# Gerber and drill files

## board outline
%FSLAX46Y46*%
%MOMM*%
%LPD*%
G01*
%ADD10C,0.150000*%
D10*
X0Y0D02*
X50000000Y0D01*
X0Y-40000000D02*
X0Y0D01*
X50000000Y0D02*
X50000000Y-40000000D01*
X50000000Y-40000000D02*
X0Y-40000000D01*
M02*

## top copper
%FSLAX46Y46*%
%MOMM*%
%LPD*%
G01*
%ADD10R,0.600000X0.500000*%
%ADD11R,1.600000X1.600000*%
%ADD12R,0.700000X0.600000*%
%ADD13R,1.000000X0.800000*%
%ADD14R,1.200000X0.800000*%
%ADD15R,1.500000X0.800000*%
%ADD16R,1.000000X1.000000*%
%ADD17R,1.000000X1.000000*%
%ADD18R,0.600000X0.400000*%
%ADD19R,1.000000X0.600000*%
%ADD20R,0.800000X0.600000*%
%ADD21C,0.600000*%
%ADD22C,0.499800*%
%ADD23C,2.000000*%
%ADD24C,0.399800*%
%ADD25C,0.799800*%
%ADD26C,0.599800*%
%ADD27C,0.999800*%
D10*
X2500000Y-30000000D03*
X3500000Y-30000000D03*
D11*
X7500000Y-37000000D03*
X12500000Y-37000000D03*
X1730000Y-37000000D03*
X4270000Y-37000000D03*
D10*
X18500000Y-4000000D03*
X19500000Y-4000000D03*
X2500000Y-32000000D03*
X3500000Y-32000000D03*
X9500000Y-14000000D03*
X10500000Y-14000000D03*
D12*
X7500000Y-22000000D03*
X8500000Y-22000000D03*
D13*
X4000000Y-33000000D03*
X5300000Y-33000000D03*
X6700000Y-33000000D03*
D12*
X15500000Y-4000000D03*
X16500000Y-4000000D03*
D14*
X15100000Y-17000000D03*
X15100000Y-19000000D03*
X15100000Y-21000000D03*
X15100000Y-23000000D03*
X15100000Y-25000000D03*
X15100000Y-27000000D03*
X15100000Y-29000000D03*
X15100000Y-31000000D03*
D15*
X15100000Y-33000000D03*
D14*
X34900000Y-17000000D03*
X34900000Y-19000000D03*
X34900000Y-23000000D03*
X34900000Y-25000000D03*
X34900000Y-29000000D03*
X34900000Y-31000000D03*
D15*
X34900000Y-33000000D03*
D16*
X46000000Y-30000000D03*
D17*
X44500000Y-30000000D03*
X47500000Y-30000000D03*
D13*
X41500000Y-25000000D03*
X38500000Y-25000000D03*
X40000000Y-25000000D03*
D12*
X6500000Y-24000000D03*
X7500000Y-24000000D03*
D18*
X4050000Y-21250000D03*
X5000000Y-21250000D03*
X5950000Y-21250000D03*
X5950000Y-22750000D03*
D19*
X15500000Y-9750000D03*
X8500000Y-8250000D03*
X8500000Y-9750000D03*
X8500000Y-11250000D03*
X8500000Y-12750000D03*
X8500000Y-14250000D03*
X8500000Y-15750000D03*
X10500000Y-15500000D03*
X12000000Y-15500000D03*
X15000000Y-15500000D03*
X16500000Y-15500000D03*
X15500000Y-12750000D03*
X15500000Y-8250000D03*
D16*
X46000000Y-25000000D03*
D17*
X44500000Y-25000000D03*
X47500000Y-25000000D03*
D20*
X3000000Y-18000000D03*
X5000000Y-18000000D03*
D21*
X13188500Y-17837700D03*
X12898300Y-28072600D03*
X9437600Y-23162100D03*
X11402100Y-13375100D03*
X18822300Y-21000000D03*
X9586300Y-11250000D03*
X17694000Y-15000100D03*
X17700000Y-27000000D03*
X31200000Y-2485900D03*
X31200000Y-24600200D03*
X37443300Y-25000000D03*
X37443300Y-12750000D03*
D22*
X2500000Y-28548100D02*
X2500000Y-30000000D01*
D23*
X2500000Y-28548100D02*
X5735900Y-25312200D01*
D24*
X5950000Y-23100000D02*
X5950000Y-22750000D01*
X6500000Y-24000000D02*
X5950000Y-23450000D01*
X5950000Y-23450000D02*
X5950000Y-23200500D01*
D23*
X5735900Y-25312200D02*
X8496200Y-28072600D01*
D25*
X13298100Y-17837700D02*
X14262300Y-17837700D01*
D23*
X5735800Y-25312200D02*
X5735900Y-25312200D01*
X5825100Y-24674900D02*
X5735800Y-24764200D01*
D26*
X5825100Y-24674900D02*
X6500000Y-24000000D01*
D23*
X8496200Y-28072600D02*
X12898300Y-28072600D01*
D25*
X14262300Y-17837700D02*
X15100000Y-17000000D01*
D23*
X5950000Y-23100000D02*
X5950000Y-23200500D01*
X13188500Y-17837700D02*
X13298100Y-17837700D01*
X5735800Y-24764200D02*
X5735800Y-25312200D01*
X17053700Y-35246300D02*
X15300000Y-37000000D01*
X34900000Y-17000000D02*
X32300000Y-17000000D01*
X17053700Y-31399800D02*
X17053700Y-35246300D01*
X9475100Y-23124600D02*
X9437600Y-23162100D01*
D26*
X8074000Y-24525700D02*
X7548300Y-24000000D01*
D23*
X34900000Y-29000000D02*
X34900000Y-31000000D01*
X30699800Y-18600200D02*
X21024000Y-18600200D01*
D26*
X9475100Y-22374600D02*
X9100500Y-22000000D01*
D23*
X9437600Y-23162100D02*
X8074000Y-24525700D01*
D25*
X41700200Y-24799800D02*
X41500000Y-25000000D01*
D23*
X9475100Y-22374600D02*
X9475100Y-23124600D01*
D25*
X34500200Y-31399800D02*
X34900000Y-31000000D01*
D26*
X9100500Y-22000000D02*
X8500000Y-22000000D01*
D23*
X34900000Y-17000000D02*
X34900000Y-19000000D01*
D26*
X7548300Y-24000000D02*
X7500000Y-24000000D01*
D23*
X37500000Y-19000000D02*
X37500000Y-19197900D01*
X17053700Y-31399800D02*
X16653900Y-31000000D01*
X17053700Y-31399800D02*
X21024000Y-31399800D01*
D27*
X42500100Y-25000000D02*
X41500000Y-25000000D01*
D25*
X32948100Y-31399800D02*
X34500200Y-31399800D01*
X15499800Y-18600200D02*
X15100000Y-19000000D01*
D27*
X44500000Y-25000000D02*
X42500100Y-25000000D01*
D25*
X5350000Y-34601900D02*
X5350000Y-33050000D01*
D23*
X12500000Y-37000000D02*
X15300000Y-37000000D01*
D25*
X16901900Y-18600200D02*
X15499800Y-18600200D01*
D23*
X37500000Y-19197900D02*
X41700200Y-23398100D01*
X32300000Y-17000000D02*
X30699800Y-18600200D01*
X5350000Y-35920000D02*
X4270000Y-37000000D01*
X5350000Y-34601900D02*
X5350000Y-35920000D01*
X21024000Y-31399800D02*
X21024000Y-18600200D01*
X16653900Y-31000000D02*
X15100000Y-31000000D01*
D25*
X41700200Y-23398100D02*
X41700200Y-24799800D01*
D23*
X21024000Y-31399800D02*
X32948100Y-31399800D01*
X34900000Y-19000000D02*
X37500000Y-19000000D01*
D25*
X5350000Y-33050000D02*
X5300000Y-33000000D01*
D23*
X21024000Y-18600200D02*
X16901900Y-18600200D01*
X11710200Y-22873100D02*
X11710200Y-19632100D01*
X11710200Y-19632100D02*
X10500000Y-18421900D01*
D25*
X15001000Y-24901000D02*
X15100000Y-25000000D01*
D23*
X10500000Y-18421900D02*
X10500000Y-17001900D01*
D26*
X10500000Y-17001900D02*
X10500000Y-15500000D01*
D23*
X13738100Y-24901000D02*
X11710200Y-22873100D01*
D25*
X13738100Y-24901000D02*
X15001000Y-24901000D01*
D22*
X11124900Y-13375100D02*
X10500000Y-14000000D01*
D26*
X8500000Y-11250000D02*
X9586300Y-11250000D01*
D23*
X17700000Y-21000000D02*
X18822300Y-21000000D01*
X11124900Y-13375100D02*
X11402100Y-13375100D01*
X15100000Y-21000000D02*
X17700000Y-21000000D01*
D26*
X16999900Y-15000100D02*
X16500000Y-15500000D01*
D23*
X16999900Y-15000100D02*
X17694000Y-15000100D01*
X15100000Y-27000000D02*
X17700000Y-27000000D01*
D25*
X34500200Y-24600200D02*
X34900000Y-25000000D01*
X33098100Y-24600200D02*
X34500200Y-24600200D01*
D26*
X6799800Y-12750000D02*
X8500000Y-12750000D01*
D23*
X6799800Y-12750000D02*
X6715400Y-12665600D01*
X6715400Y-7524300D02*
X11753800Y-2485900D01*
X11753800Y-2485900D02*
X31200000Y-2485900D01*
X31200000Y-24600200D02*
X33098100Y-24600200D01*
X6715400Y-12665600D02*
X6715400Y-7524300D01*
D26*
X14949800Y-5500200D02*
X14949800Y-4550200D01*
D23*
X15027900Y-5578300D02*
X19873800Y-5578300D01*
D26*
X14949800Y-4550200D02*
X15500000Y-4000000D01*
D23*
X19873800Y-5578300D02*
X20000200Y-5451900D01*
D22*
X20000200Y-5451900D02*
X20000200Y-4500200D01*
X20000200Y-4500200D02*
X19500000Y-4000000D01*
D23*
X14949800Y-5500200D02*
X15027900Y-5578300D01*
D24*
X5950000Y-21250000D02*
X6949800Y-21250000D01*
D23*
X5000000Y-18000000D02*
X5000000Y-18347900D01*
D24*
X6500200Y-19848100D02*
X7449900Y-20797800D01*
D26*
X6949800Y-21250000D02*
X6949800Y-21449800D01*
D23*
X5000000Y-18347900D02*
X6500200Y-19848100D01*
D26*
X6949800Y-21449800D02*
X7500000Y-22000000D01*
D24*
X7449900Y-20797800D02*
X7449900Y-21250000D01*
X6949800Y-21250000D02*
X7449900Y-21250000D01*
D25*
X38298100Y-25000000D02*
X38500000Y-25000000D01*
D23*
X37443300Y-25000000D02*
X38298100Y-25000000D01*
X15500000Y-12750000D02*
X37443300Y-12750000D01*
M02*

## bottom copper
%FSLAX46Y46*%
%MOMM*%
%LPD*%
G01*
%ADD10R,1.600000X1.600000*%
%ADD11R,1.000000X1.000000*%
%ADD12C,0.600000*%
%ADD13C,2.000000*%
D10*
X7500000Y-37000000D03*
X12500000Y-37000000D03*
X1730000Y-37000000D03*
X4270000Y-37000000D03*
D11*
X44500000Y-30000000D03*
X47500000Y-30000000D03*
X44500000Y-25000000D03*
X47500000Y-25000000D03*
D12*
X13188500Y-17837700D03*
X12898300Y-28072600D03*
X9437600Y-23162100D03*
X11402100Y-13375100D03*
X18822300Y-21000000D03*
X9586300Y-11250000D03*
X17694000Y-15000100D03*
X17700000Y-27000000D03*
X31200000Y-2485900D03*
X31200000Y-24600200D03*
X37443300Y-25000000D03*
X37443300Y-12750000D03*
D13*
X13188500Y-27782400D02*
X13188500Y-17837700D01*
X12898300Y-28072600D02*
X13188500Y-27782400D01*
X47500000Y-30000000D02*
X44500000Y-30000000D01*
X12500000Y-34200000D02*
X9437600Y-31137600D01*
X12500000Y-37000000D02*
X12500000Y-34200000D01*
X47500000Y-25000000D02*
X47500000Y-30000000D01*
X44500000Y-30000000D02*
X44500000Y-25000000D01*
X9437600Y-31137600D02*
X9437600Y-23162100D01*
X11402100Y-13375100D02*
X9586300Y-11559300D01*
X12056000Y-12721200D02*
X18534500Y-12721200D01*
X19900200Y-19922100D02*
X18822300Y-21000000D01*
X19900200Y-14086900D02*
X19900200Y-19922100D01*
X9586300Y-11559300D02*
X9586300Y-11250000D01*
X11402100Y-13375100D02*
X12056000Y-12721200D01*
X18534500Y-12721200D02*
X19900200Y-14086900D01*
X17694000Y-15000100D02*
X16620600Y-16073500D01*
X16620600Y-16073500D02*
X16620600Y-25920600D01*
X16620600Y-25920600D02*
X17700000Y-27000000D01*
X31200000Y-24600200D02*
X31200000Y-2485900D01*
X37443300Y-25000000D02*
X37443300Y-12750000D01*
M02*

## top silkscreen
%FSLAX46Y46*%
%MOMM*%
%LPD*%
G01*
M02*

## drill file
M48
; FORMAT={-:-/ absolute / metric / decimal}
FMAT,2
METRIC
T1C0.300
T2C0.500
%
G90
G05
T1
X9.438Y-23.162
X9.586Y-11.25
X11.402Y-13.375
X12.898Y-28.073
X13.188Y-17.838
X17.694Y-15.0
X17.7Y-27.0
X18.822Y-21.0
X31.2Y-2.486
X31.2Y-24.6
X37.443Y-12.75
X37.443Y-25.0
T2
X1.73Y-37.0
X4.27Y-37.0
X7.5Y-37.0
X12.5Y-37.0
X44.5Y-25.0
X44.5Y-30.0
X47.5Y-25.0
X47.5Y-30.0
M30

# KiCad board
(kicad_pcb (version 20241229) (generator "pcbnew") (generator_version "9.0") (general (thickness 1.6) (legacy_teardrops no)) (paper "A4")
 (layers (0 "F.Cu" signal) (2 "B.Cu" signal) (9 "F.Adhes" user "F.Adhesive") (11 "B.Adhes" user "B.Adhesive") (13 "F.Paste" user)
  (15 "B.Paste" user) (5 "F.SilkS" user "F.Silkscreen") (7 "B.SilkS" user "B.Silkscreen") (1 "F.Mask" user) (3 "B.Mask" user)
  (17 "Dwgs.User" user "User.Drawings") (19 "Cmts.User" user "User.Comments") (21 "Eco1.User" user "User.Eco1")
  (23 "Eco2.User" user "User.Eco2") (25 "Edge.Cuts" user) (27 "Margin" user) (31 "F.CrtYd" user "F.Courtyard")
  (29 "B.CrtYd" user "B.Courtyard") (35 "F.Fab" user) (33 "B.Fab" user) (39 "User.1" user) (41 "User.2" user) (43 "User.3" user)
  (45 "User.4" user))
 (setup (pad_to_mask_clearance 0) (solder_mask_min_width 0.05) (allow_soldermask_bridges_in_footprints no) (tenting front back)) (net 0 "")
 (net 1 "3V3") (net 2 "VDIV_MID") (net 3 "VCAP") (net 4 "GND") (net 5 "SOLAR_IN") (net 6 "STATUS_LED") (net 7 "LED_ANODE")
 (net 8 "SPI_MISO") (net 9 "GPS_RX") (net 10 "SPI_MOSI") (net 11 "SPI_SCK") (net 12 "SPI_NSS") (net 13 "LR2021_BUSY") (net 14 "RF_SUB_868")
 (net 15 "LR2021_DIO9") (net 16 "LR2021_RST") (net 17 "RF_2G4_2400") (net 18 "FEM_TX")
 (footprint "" (layer "F.Cu") (at 3 30)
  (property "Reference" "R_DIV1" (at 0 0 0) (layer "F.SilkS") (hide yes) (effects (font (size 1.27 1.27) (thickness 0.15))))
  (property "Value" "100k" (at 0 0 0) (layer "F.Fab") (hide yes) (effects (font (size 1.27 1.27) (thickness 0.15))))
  (pad "1" smd rect (at -0.5 0) (size 0.6 0.5) (layers "F.Cu" "F.Mask") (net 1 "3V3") (thermal_bridge_angle 45))
  (pad "2" smd rect (at 0.5 0) (size 0.6 0.5) (layers "F.Cu" "F.Mask") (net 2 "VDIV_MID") (thermal_bridge_angle 45)))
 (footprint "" (layer "F.Cu") (at 10 37)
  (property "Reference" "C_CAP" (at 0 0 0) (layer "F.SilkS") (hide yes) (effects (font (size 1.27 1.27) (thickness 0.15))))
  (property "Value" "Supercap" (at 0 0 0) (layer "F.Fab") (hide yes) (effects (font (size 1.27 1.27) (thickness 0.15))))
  (pad "1" thru_hole rect (at -2.5 0) (size 1.6 1.6) (drill 0.5) (layers "*.Cu" "*.Mask") (remove_unused_layers no) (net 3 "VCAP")
   (thermal_bridge_angle 45))
  (pad "2" thru_hole rect (at 2.5 0) (size 1.6 1.6) (drill 0.5) (layers "*.Cu" "*.Mask") (remove_unused_layers no) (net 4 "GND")
   (thermal_bridge_angle 45)))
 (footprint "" (layer "F.Cu") (at 3 37)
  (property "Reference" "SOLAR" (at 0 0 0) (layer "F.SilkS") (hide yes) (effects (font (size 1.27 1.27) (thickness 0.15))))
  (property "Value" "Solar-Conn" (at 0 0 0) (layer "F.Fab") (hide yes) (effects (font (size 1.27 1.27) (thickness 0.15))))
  (pad "1" thru_hole rect (at -1.27 0) (size 1.6 1.6) (drill 0.5) (layers "*.Cu" "*.Mask") (remove_unused_layers no) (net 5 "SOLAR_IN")
   (thermal_bridge_angle 45))
  (pad "2" thru_hole rect (at 1.27 0) (size 1.6 1.6) (drill 0.5) (layers "*.Cu" "*.Mask") (remove_unused_layers no) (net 4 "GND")
   (thermal_bridge_angle 45)))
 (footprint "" (layer "F.Cu") (at 19 4)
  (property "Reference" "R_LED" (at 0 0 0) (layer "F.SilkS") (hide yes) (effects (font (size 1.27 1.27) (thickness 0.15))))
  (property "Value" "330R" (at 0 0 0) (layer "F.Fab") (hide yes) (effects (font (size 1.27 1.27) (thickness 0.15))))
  (pad "1" smd rect (at -0.5 0) (size 0.6 0.5) (layers "F.Cu" "F.Mask") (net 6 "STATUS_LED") (thermal_bridge_angle 45))
  (pad "2" smd rect (at 0.5 0) (size 0.6 0.5) (layers "F.Cu" "F.Mask") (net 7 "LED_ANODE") (thermal_bridge_angle 45)))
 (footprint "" (layer "F.Cu") (at 3 32)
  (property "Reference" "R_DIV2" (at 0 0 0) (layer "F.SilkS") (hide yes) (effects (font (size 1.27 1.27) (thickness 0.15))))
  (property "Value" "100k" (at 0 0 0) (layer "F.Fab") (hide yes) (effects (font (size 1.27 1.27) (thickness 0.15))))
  (pad "1" smd rect (at -0.5 0) (size 0.6 0.5) (layers "F.Cu" "F.Mask") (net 2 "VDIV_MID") (thermal_bridge_angle 45))
  (pad "2" smd rect (at 0.5 0) (size 0.6 0.5) (layers "F.Cu" "F.Mask") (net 4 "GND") (thermal_bridge_angle 45)))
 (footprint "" (layer "F.Cu") (at 10 14)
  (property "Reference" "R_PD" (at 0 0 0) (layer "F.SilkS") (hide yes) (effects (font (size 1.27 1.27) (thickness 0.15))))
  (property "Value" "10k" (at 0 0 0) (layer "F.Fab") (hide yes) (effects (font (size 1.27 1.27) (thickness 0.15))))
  (pad "1" smd rect (at -0.5 0) (size 0.6 0.5) (layers "F.Cu" "F.Mask") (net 4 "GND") (thermal_bridge_angle 45))
  (pad "2" smd rect (at 0.5 0) (size 0.6 0.5) (layers "F.Cu" "F.Mask") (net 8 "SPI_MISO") (thermal_bridge_angle 45)))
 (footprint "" (layer "F.Cu") (at 8 22)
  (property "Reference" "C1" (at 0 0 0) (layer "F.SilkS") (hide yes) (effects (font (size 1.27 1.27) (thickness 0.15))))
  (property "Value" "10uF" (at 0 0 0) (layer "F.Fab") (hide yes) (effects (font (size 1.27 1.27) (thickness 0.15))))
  (pad "1" smd rect (at -0.5 0) (size 0.7 0.6) (layers "F.Cu" "F.Mask") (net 3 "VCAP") (thermal_bridge_angle 45))
  (pad "2" smd rect (at 0.5 0) (size 0.7 0.6) (layers "F.Cu" "F.Mask") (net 4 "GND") (thermal_bridge_angle 45)))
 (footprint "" (layer "F.Cu") (at 6 33)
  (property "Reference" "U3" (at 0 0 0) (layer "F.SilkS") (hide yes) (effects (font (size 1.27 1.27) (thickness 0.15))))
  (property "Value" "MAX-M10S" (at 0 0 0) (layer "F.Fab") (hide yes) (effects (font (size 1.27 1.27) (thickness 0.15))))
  (pad "1" smd rect (at -2 0) (size 1 0.8) (layers "F.Cu" "F.Mask") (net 1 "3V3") (thermal_bridge_angle 45))
  (pad "2" smd rect (at -0.7 0) (size 1 0.8) (layers "F.Cu" "F.Mask") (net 4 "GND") (thermal_bridge_angle 45))
  (pad "3" smd rect (at 0.7 0) (size 1 0.8) (layers "F.Cu" "F.Mask") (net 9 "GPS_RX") (thermal_bridge_angle 45)))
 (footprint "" (layer "F.Cu") (at 16 4)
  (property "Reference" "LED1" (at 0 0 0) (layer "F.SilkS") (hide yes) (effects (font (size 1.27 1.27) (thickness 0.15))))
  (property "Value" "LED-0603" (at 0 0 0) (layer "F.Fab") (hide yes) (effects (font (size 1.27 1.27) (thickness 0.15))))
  (pad "A" smd rect (at -0.5 0) (size 0.7 0.6) (layers "F.Cu" "F.Mask") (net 7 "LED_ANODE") (thermal_bridge_angle 45))
  (pad "K" smd rect (at 0.5 0) (size 0.7 0.6) (layers "F.Cu" "F.Mask") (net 4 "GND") (thermal_bridge_angle 45)))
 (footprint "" (layer "F.Cu") (at 25 25)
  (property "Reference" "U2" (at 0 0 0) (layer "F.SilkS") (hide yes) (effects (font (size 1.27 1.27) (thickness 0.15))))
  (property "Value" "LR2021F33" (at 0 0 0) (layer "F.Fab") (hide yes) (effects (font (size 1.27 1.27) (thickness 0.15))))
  (pad "1" smd rect (at -9.9 -8) (size 1.2 0.8) (layers "F.Cu" "F.Mask") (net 1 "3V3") (thermal_bridge_angle 45))
  (pad "2" smd rect (at -9.9 -6) (size 1.2 0.8) (layers "F.Cu" "F.Mask") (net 4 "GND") (thermal_bridge_angle 45))
  (pad "3" smd rect (at -9.9 -4) (size 1.2 0.8) (layers "F.Cu" "F.Mask") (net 8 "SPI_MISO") (thermal_bridge_angle 45))
  (pad "4" smd rect (at -9.9 -2) (size 1.2 0.8) (layers "F.Cu" "F.Mask") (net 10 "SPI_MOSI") (thermal_bridge_angle 45))
  (pad "5" smd rect (at -9.9 0) (size 1.2 0.8) (layers "F.Cu" "F.Mask") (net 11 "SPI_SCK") (thermal_bridge_angle 45))
  (pad "6" smd rect (at -9.9 2) (size 1.2 0.8) (layers "F.Cu" "F.Mask") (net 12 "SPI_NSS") (thermal_bridge_angle 45))
  (pad "7" smd rect (at -9.9 4) (size 1.2 0.8) (layers "F.Cu" "F.Mask") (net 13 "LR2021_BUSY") (thermal_bridge_angle 45))
  (pad "8" smd rect (at -9.9 6) (size 1.2 0.8) (layers "F.Cu" "F.Mask") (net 4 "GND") (thermal_bridge_angle 45))
  (pad "9" smd rect (at -9.9 8) (size 1.5 0.8) (layers "F.Cu" "F.Mask") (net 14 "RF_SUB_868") (thermal_bridge_angle 45))
  (pad "10" smd rect (at 9.9 -8) (size 1.2 0.8) (layers "F.Cu" "F.Mask") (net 4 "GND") (thermal_bridge_angle 45))
  (pad "11" smd rect (at 9.9 -6) (size 1.2 0.8) (layers "F.Cu" "F.Mask") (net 4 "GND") (thermal_bridge_angle 45))
  (pad "13" smd rect (at 9.9 -2) (size 1.2 0.8) (layers "F.Cu" "F.Mask") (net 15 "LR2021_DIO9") (thermal_bridge_angle 45))
  (pad "14" smd rect (at 9.9 0) (size 1.2 0.8) (layers "F.Cu" "F.Mask") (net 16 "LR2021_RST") (thermal_bridge_angle 45))
  (pad "16" smd rect (at 9.9 4) (size 1.2 0.8) (layers "F.Cu" "F.Mask") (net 4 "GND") (thermal_bridge_angle 45))
  (pad "17" smd rect (at 9.9 6) (size 1.2 0.8) (layers "F.Cu" "F.Mask") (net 4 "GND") (thermal_bridge_angle 45))
  (pad "18" smd rect (at 9.9 8) (size 1.5 0.8) (layers "F.Cu" "F.Mask") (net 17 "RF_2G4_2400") (thermal_bridge_angle 45)))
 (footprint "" (layer "F.Cu") (at 46 30)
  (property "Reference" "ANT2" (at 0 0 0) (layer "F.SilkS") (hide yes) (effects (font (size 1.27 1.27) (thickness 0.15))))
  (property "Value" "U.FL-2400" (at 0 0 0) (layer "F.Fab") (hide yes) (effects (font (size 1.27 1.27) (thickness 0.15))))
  (pad "1" smd rect (at 0 0) (size 1 1) (layers "F.Cu" "F.Mask") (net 17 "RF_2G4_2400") (thermal_bridge_angle 45))
  (pad "2" thru_hole rect (at -1.5 0) (size 1 1) (drill 0.5) (layers "*.Cu" "*.Mask") (remove_unused_layers no) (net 4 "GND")
   (thermal_bridge_angle 45))
  (pad "3" thru_hole rect (at 1.5 0) (size 1 1) (drill 0.5) (layers "*.Cu" "*.Mask") (remove_unused_layers no) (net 4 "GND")
   (thermal_bridge_angle 45)))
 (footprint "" (layer "F.Cu") (at 40 25)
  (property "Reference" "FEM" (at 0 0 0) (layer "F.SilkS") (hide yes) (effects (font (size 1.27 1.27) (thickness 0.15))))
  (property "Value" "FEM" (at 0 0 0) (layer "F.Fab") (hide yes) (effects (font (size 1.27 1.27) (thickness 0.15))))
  (pad "GND" smd rect (at 1.5 0) (size 1 0.8) (layers "F.Cu" "F.Mask") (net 4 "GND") (thermal_bridge_angle 45))
  (pad "TX" smd rect (at -1.5 0) (size 1 0.8) (layers "F.Cu" "F.Mask") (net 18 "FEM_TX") (thermal_bridge_angle 45))
  (pad "VCC" smd rect (at 0 0) (size 1 0.8) (layers "F.Cu" "F.Mask") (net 1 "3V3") (thermal_bridge_angle 45)))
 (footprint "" (layer "F.Cu") (at 7 24)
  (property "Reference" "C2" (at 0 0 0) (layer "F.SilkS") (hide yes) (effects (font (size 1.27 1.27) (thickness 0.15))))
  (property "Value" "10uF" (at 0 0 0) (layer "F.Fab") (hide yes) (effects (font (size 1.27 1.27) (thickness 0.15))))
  (pad "1" smd rect (at -0.5 0) (size 0.7 0.6) (layers "F.Cu" "F.Mask") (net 1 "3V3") (thermal_bridge_angle 45))
  (pad "2" smd rect (at 0.5 0) (size 0.7 0.6) (layers "F.Cu" "F.Mask") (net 4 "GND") (thermal_bridge_angle 45)))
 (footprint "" (layer "F.Cu") (at 5 22)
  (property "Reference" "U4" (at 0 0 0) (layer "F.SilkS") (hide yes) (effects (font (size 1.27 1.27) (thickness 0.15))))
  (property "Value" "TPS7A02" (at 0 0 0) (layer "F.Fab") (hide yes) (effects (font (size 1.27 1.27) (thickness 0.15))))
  (pad "1" smd rect (at -0.95 -0.75) (size 0.6 0.4) (layers "F.Cu" "F.Mask") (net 3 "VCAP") (thermal_bridge_angle 45))
  (pad "2" smd rect (at 0 -0.75) (size 0.6 0.4) (layers "F.Cu" "F.Mask") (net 4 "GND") (thermal_bridge_angle 45))
  (pad "3" smd rect (at 0.95 -0.75) (size 0.6 0.4) (layers "F.Cu" "F.Mask") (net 3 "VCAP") (thermal_bridge_angle 45))
  (pad "4" smd rect (at 0.95 0.75) (size 0.6 0.4) (layers "F.Cu" "F.Mask") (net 1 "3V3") (thermal_bridge_angle 45)))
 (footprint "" (layer "F.Cu") (at 12 12)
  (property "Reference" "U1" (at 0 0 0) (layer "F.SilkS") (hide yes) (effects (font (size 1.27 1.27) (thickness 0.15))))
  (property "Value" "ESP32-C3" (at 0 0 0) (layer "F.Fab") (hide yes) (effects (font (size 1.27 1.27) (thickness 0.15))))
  (pad "GND" smd rect (at 3.5 -2.25) (size 1 0.6) (layers "F.Cu" "F.Mask") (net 4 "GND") (thermal_bridge_angle 45))
  (pad "GPIO0" smd rect (at -3.5 -3.75) (size 1 0.6) (layers "F.Cu" "F.Mask") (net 2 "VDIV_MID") (thermal_bridge_angle 45))
  (pad "GPIO1" smd rect (at -3.5 -2.25) (size 1 0.6) (layers "F.Cu" "F.Mask") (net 9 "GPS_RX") (thermal_bridge_angle 45))
  (pad "GPIO2" smd rect (at -3.5 -0.75) (size 1 0.6) (layers "F.Cu" "F.Mask") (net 8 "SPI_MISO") (thermal_bridge_angle 45))
  (pad "GPIO3" smd rect (at -3.5 0.75) (size 1 0.6) (layers "F.Cu" "F.Mask") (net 16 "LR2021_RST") (thermal_bridge_angle 45))
  (pad "GPIO4" smd rect (at -3.5 2.25) (size 1 0.6) (layers "F.Cu" "F.Mask") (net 13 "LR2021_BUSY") (thermal_bridge_angle 45))
  (pad "GPIO5" smd rect (at -3.5 3.75) (size 1 0.6) (layers "F.Cu" "F.Mask") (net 15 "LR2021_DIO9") (thermal_bridge_angle 45))
  (pad "GPIO6" smd rect (at -1.5 3.5) (size 1 0.6) (layers "F.Cu" "F.Mask") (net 11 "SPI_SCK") (thermal_bridge_angle 45))
  (pad "GPIO7" smd rect (at 0 3.5) (size 1 0.6) (layers "F.Cu" "F.Mask") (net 10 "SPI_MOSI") (thermal_bridge_angle 45))
  (pad "GPIO9" smd rect (at 3 3.5) (size 1 0.6) (layers "F.Cu" "F.Mask") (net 6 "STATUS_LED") (thermal_bridge_angle 45))
  (pad "GPIO10" smd rect (at 4.5 3.5) (size 1 0.6) (layers "F.Cu" "F.Mask") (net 12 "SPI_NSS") (thermal_bridge_angle 45))
  (pad "GPIO19" smd rect (at 3.5 0.75) (size 1 0.6) (layers "F.Cu" "F.Mask") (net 18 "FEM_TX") (thermal_bridge_angle 45))
  (pad "VCC" smd rect (at 3.5 -3.75) (size 1 0.6) (layers "F.Cu" "F.Mask") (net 1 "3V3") (thermal_bridge_angle 45)))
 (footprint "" (layer "F.Cu") (at 46 25)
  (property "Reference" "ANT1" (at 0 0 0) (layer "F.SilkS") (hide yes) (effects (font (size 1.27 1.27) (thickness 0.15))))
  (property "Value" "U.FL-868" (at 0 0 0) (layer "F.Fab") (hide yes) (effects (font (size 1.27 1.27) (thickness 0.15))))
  (pad "1" smd rect (at 0 0) (size 1 1) (layers "F.Cu" "F.Mask") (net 14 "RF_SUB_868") (thermal_bridge_angle 45))
  (pad "2" thru_hole rect (at -1.5 0) (size 1 1) (drill 0.5) (layers "*.Cu" "*.Mask") (remove_unused_layers no) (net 4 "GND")
   (thermal_bridge_angle 45))
  (pad "3" thru_hole rect (at 1.5 0) (size 1 1) (drill 0.5) (layers "*.Cu" "*.Mask") (remove_unused_layers no) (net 4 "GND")
   (thermal_bridge_angle 45)))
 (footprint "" (layer "F.Cu") (at 4 18)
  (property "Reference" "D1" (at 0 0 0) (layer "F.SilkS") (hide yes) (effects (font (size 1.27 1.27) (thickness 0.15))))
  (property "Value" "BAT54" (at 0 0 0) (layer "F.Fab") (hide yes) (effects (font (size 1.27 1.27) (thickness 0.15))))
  (pad "A" smd rect (at -1 0) (size 0.8 0.6) (layers "F.Cu" "F.Mask") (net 5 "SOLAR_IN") (thermal_bridge_angle 45))
  (pad "K" smd rect (at 1 0) (size 0.8 0.6) (layers "F.Cu" "F.Mask") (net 3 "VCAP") (thermal_bridge_angle 45)))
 (gr_line (start 0 0) (end 50 0) (stroke (width 0.15) (type default)) (layer "Edge.Cuts"))
 (gr_line (start 0 40) (end 0 0) (stroke (width 0.15) (type default)) (layer "Edge.Cuts"))
 (gr_line (start 50 0) (end 50 40) (stroke (width 0.15) (type default)) (layer "Edge.Cuts"))
 (gr_line (start 50 40) (end 0 40) (stroke (width 0.15) (type default)) (layer "Edge.Cuts"))
 (segment (start 2.5 28.5481) (end 2.5 30) (width 0.4998) (layer "F.Cu") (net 1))
 (segment (start 2.5 28.5481) (end 5.7359 25.3122) (width 2) (layer "F.Cu") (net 1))
 (segment (start 5.95 23.1) (end 5.95 22.75) (width 0.3998) (layer "F.Cu") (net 1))
 (segment (start 6.5 24) (end 5.95 23.45) (width 0.3998) (layer "F.Cu") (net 1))
 (segment (start 5.95 23.45) (end 5.95 23.2005) (width 0.3998) (layer "F.Cu") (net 1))
 (segment (start 5.7359 25.3122) (end 8.4962 28.0726) (width 2) (layer "F.Cu") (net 1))
 (segment (start 13.2981 17.8377) (end 14.2623 17.8377) (width 0.7998) (layer "F.Cu") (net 1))
 (segment (start 5.7358 25.3122) (end 5.7359 25.3122) (width 2) (layer "F.Cu") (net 1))
 (segment (start 5.8251 24.6749) (end 5.7358 24.7642) (width 2) (layer "F.Cu") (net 1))
 (segment (start 5.8251 24.6749) (end 6.5 24) (width 0.5998) (layer "F.Cu") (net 1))
 (segment (start 8.4962 28.0726) (end 12.8983 28.0726) (width 2) (layer "F.Cu") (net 1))
 (segment (start 14.2623 17.8377) (end 15.1 17) (width 0.7998) (layer "F.Cu") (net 1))
 (segment (start 5.95 23.1) (end 5.95 23.2005) (width 2) (layer "F.Cu") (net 1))
 (segment (start 13.1885 17.8377) (end 13.2981 17.8377) (width 2) (layer "F.Cu") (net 1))
 (segment (start 5.7358 24.7642) (end 5.7358 25.3122) (width 2) (layer "F.Cu") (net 1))
 (via (at 13.1885 17.8377) (size 0.6) (drill 0.3) (layers "F.Cu" "B.Cu") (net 1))
 (via (at 12.8983 28.0726) (size 0.6) (drill 0.3) (layers "F.Cu" "B.Cu") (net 1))
 (segment (start 13.1885 27.7824) (end 13.1885 17.8377) (width 2) (layer "B.Cu") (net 1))
 (segment (start 12.8983 28.0726) (end 13.1885 27.7824) (width 2) (layer "B.Cu") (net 1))
 (segment (start 17.0537 35.2463) (end 15.3 37) (width 2) (layer "F.Cu") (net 4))
 (segment (start 34.9 17) (end 32.3 17) (width 2) (layer "F.Cu") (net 4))
 (segment (start 17.0537 31.3998) (end 17.0537 35.2463) (width 2) (layer "F.Cu") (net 4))
 (segment (start 9.4751 23.1246) (end 9.4376 23.1621) (width 2) (layer "F.Cu") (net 4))
 (segment (start 8.074 24.5257) (end 7.5483 24) (width 0.5998) (layer "F.Cu") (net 4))
 (segment (start 34.9 29) (end 34.9 31) (width 2) (layer "F.Cu") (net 4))
 (segment (start 30.6998 18.6002) (end 21.024 18.6002) (width 2) (layer "F.Cu") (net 4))
 (segment (start 9.4751 22.3746) (end 9.1005 22) (width 0.5998) (layer "F.Cu") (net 4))
 (segment (start 9.4376 23.1621) (end 8.074 24.5257) (width 2) (layer "F.Cu") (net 4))
 (segment (start 41.7002 24.7998) (end 41.5 25) (width 0.7998) (layer "F.Cu") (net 4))
 (segment (start 9.4751 22.3746) (end 9.4751 23.1246) (width 2) (layer "F.Cu") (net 4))
 (segment (start 34.5002 31.3998) (end 34.9 31) (width 0.7998) (layer "F.Cu") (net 4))
 (segment (start 9.1005 22) (end 8.5 22) (width 0.5998) (layer "F.Cu") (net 4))
 (segment (start 34.9 17) (end 34.9 19) (width 2) (layer "F.Cu") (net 4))
 (segment (start 7.5483 24) (end 7.5 24) (width 0.5998) (layer "F.Cu") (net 4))
 (segment (start 37.5 19) (end 37.5 19.1979) (width 2) (layer "F.Cu") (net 4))
 (segment (start 17.0537 31.3998) (end 16.6539 31) (width 2) (layer "F.Cu") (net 4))
 (segment (start 17.0537 31.3998) (end 21.024 31.3998) (width 2) (layer "F.Cu") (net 4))
 (segment (start 42.5001 25) (end 41.5 25) (width 0.9998) (layer "F.Cu") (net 4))
 (segment (start 32.9481 31.3998) (end 34.5002 31.3998) (width 0.7998) (layer "F.Cu") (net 4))
 (segment (start 15.4998 18.6002) (end 15.1 19) (width 0.7998) (layer "F.Cu") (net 4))
 (segment (start 44.5 25) (end 42.5001 25) (width 0.9998) (layer "F.Cu") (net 4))
 (segment (start 5.35 34.6019) (end 5.35 33.05) (width 0.7998) (layer "F.Cu") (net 4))
 (segment (start 12.5 37) (end 15.3 37) (width 2) (layer "F.Cu") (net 4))
 (segment (start 16.9019 18.6002) (end 15.4998 18.6002) (width 0.7998) (layer "F.Cu") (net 4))
 (segment (start 37.5 19.1979) (end 41.7002 23.3981) (width 2) (layer "F.Cu") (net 4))
 (segment (start 32.3 17) (end 30.6998 18.6002) (width 2) (layer "F.Cu") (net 4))
 (segment (start 5.35 35.92) (end 4.27 37) (width 2) (layer "F.Cu") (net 4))
 (segment (start 5.35 34.6019) (end 5.35 35.92) (width 2) (layer "F.Cu") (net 4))
 (segment (start 21.024 31.3998) (end 21.024 18.6002) (width 2) (layer "F.Cu") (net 4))
 (segment (start 16.6539 31) (end 15.1 31) (width 2) (layer "F.Cu") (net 4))
 (segment (start 41.7002 23.3981) (end 41.7002 24.7998) (width 0.7998) (layer "F.Cu") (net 4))
 (segment (start 21.024 31.3998) (end 32.9481 31.3998) (width 2) (layer "F.Cu") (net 4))
 (segment (start 34.9 19) (end 37.5 19) (width 2) (layer "F.Cu") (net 4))
 (segment (start 5.35 33.05) (end 5.3 33) (width 0.7998) (layer "F.Cu") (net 4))
 (segment (start 21.024 18.6002) (end 16.9019 18.6002) (width 2) (layer "F.Cu") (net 4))
 (via (at 9.4376 23.1621) (size 0.6) (drill 0.3) (layers "F.Cu" "B.Cu") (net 4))
 (segment (start 47.5 30) (end 44.5 30) (width 2) (layer "B.Cu") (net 4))
 (segment (start 12.5 34.2) (end 9.4376 31.1376) (width 2) (layer "B.Cu") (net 4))
 (segment (start 12.5 37) (end 12.5 34.2) (width 2) (layer "B.Cu") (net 4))
 (segment (start 47.5 25) (end 47.5 30) (width 2) (layer "B.Cu") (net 4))
 (segment (start 44.5 30) (end 44.5 25) (width 2) (layer "B.Cu") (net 4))
 (segment (start 9.4376 31.1376) (end 9.4376 23.1621) (width 2) (layer "B.Cu") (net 4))
 (segment (start 11.7102 22.8731) (end 11.7102 19.6321) (width 2) (layer "F.Cu") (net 11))
 (segment (start 11.7102 19.6321) (end 10.5 18.4219) (width 2) (layer "F.Cu") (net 11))
 (segment (start 15.001 24.901) (end 15.1 25) (width 0.7998) (layer "F.Cu") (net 11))
 (segment (start 10.5 18.4219) (end 10.5 17.0019) (width 2) (layer "F.Cu") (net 11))
 (segment (start 10.5 17.0019) (end 10.5 15.5) (width 0.5998) (layer "F.Cu") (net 11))
 (segment (start 13.7381 24.901) (end 11.7102 22.8731) (width 2) (layer "F.Cu") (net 11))
 (segment (start 13.7381 24.901) (end 15.001 24.901) (width 0.7998) (layer "F.Cu") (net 11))
 (segment (start 11.1249 13.3751) (end 10.5 14) (width 0.4998) (layer "F.Cu") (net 8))
 (segment (start 8.5 11.25) (end 9.5863 11.25) (width 0.5998) (layer "F.Cu") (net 8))
 (segment (start 17.7 21) (end 18.8223 21) (width 2) (layer "F.Cu") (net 8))
 (segment (start 11.1249 13.3751) (end 11.4021 13.3751) (width 2) (layer "F.Cu") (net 8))
 (segment (start 15.1 21) (end 17.7 21) (width 2) (layer "F.Cu") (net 8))
 (via (at 11.4021 13.3751) (size 0.6) (drill 0.3) (layers "F.Cu" "B.Cu") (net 8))
 (via (at 18.8223 21) (size 0.6) (drill 0.3) (layers "F.Cu" "B.Cu") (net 8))
 (via (at 9.5863 11.25) (size 0.6) (drill 0.3) (layers "F.Cu" "B.Cu") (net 8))
 (segment (start 11.4021 13.3751) (end 9.5863 11.5593) (width 2) (layer "B.Cu") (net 8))
 (segment (start 12.056 12.7212) (end 18.5345 12.7212) (width 2) (layer "B.Cu") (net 8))
 (segment (start 19.9002 19.9221) (end 18.8223 21) (width 2) (layer "B.Cu") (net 8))
 (segment (start 19.9002 14.0869) (end 19.9002 19.9221) (width 2) (layer "B.Cu") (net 8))
 (segment (start 9.5863 11.5593) (end 9.5863 11.25) (width 2) (layer "B.Cu") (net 8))
 (segment (start 11.4021 13.3751) (end 12.056 12.7212) (width 2) (layer "B.Cu") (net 8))
 (segment (start 18.5345 12.7212) (end 19.9002 14.0869) (width 2) (layer "B.Cu") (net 8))
 (segment (start 16.9999 15.0001) (end 16.5 15.5) (width 0.5998) (layer "F.Cu") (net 12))
 (segment (start 16.9999 15.0001) (end 17.694 15.0001) (width 2) (layer "F.Cu") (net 12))
 (segment (start 15.1 27) (end 17.7 27) (width 2) (layer "F.Cu") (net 12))
 (via (at 17.694 15.0001) (size 0.6) (drill 0.3) (layers "F.Cu" "B.Cu") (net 12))
 (via (at 17.7 27) (size 0.6) (drill 0.3) (layers "F.Cu" "B.Cu") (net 12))
 (segment (start 17.694 15.0001) (end 16.6206 16.0735) (width 2) (layer "B.Cu") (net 12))
 (segment (start 16.6206 16.0735) (end 16.6206 25.9206) (width 2) (layer "B.Cu") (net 12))
 (segment (start 16.6206 25.9206) (end 17.7 27) (width 2) (layer "B.Cu") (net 12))
 (segment (start 34.5002 24.6002) (end 34.9 25) (width 0.7998) (layer "F.Cu") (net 16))
 (segment (start 33.0981 24.6002) (end 34.5002 24.6002) (width 0.7998) (layer "F.Cu") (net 16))
 (segment (start 6.7998 12.75) (end 8.5 12.75) (width 0.5998) (layer "F.Cu") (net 16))
 (segment (start 6.7998 12.75) (end 6.7154 12.6656) (width 2) (layer "F.Cu") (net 16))
 (segment (start 6.7154 7.5243) (end 11.7538 2.4859) (width 2) (layer "F.Cu") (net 16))
 (segment (start 11.7538 2.4859) (end 31.2 2.4859) (width 2) (layer "F.Cu") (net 16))
 (segment (start 31.2 24.6002) (end 33.0981 24.6002) (width 2) (layer "F.Cu") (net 16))
 (segment (start 6.7154 12.6656) (end 6.7154 7.5243) (width 2) (layer "F.Cu") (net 16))
 (via (at 31.2 2.4859) (size 0.6) (drill 0.3) (layers "F.Cu" "B.Cu") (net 16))
 (via (at 31.2 24.6002) (size 0.6) (drill 0.3) (layers "F.Cu" "B.Cu") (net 16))
 (segment (start 31.2 24.6002) (end 31.2 2.4859) (width 2) (layer "B.Cu") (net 16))
 (segment (start 14.9498 5.5002) (end 14.9498 4.5502) (width 0.5998) (layer "F.Cu") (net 7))
 (segment (start 15.0279 5.5783) (end 19.8738 5.5783) (width 2) (layer "F.Cu") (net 7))
 (segment (start 14.9498 4.5502) (end 15.5 4) (width 0.5998) (layer "F.Cu") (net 7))
 (segment (start 19.8738 5.5783) (end 20.0002 5.4519) (width 2) (layer "F.Cu") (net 7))
 (segment (start 20.0002 5.4519) (end 20.0002 4.5002) (width 0.4998) (layer "F.Cu") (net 7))
 (segment (start 20.0002 4.5002) (end 19.5 4) (width 0.4998) (layer "F.Cu") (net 7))
 (segment (start 14.9498 5.5002) (end 15.0279 5.5783) (width 2) (layer "F.Cu") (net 7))
 (segment (start 5.95 21.25) (end 6.9498 21.25) (width 0.3998) (layer "F.Cu") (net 3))
 (segment (start 5 18) (end 5 18.3479) (width 2) (layer "F.Cu") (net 3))
 (segment (start 6.5002 19.8481) (end 7.4499 20.7978) (width 0.3998) (layer "F.Cu") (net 3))
 (segment (start 6.9498 21.25) (end 6.9498 21.4498) (width 0.5998) (layer "F.Cu") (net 3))
 (segment (start 5 18.3479) (end 6.5002 19.8481) (width 2) (layer "F.Cu") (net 3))
 (segment (start 6.9498 21.4498) (end 7.5 22) (width 0.5998) (layer "F.Cu") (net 3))
 (segment (start 7.4499 20.7978) (end 7.4499 21.25) (width 0.3998) (layer "F.Cu") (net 3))
 (segment (start 6.9498 21.25) (end 7.4499 21.25) (width 0.3998) (layer "F.Cu") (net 3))
 (segment (start 38.2981 25) (end 38.5 25) (width 0.7998) (layer "F.Cu") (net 18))
 (segment (start 37.4433 25) (end 38.2981 25) (width 2) (layer "F.Cu") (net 18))
 (segment (start 15.5 12.75) (end 37.4433 12.75) (width 2) (layer "F.Cu") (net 18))
 (via (at 37.4433 25) (size 0.6) (drill 0.3) (layers "F.Cu" "B.Cu") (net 18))
 (via (at 37.4433 12.75) (size 0.6) (drill 0.3) (layers "F.Cu" "B.Cu") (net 18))
 (segment (start 37.4433 25) (end 37.4433 12.75) (width 2) (layer "B.Cu") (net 18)))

